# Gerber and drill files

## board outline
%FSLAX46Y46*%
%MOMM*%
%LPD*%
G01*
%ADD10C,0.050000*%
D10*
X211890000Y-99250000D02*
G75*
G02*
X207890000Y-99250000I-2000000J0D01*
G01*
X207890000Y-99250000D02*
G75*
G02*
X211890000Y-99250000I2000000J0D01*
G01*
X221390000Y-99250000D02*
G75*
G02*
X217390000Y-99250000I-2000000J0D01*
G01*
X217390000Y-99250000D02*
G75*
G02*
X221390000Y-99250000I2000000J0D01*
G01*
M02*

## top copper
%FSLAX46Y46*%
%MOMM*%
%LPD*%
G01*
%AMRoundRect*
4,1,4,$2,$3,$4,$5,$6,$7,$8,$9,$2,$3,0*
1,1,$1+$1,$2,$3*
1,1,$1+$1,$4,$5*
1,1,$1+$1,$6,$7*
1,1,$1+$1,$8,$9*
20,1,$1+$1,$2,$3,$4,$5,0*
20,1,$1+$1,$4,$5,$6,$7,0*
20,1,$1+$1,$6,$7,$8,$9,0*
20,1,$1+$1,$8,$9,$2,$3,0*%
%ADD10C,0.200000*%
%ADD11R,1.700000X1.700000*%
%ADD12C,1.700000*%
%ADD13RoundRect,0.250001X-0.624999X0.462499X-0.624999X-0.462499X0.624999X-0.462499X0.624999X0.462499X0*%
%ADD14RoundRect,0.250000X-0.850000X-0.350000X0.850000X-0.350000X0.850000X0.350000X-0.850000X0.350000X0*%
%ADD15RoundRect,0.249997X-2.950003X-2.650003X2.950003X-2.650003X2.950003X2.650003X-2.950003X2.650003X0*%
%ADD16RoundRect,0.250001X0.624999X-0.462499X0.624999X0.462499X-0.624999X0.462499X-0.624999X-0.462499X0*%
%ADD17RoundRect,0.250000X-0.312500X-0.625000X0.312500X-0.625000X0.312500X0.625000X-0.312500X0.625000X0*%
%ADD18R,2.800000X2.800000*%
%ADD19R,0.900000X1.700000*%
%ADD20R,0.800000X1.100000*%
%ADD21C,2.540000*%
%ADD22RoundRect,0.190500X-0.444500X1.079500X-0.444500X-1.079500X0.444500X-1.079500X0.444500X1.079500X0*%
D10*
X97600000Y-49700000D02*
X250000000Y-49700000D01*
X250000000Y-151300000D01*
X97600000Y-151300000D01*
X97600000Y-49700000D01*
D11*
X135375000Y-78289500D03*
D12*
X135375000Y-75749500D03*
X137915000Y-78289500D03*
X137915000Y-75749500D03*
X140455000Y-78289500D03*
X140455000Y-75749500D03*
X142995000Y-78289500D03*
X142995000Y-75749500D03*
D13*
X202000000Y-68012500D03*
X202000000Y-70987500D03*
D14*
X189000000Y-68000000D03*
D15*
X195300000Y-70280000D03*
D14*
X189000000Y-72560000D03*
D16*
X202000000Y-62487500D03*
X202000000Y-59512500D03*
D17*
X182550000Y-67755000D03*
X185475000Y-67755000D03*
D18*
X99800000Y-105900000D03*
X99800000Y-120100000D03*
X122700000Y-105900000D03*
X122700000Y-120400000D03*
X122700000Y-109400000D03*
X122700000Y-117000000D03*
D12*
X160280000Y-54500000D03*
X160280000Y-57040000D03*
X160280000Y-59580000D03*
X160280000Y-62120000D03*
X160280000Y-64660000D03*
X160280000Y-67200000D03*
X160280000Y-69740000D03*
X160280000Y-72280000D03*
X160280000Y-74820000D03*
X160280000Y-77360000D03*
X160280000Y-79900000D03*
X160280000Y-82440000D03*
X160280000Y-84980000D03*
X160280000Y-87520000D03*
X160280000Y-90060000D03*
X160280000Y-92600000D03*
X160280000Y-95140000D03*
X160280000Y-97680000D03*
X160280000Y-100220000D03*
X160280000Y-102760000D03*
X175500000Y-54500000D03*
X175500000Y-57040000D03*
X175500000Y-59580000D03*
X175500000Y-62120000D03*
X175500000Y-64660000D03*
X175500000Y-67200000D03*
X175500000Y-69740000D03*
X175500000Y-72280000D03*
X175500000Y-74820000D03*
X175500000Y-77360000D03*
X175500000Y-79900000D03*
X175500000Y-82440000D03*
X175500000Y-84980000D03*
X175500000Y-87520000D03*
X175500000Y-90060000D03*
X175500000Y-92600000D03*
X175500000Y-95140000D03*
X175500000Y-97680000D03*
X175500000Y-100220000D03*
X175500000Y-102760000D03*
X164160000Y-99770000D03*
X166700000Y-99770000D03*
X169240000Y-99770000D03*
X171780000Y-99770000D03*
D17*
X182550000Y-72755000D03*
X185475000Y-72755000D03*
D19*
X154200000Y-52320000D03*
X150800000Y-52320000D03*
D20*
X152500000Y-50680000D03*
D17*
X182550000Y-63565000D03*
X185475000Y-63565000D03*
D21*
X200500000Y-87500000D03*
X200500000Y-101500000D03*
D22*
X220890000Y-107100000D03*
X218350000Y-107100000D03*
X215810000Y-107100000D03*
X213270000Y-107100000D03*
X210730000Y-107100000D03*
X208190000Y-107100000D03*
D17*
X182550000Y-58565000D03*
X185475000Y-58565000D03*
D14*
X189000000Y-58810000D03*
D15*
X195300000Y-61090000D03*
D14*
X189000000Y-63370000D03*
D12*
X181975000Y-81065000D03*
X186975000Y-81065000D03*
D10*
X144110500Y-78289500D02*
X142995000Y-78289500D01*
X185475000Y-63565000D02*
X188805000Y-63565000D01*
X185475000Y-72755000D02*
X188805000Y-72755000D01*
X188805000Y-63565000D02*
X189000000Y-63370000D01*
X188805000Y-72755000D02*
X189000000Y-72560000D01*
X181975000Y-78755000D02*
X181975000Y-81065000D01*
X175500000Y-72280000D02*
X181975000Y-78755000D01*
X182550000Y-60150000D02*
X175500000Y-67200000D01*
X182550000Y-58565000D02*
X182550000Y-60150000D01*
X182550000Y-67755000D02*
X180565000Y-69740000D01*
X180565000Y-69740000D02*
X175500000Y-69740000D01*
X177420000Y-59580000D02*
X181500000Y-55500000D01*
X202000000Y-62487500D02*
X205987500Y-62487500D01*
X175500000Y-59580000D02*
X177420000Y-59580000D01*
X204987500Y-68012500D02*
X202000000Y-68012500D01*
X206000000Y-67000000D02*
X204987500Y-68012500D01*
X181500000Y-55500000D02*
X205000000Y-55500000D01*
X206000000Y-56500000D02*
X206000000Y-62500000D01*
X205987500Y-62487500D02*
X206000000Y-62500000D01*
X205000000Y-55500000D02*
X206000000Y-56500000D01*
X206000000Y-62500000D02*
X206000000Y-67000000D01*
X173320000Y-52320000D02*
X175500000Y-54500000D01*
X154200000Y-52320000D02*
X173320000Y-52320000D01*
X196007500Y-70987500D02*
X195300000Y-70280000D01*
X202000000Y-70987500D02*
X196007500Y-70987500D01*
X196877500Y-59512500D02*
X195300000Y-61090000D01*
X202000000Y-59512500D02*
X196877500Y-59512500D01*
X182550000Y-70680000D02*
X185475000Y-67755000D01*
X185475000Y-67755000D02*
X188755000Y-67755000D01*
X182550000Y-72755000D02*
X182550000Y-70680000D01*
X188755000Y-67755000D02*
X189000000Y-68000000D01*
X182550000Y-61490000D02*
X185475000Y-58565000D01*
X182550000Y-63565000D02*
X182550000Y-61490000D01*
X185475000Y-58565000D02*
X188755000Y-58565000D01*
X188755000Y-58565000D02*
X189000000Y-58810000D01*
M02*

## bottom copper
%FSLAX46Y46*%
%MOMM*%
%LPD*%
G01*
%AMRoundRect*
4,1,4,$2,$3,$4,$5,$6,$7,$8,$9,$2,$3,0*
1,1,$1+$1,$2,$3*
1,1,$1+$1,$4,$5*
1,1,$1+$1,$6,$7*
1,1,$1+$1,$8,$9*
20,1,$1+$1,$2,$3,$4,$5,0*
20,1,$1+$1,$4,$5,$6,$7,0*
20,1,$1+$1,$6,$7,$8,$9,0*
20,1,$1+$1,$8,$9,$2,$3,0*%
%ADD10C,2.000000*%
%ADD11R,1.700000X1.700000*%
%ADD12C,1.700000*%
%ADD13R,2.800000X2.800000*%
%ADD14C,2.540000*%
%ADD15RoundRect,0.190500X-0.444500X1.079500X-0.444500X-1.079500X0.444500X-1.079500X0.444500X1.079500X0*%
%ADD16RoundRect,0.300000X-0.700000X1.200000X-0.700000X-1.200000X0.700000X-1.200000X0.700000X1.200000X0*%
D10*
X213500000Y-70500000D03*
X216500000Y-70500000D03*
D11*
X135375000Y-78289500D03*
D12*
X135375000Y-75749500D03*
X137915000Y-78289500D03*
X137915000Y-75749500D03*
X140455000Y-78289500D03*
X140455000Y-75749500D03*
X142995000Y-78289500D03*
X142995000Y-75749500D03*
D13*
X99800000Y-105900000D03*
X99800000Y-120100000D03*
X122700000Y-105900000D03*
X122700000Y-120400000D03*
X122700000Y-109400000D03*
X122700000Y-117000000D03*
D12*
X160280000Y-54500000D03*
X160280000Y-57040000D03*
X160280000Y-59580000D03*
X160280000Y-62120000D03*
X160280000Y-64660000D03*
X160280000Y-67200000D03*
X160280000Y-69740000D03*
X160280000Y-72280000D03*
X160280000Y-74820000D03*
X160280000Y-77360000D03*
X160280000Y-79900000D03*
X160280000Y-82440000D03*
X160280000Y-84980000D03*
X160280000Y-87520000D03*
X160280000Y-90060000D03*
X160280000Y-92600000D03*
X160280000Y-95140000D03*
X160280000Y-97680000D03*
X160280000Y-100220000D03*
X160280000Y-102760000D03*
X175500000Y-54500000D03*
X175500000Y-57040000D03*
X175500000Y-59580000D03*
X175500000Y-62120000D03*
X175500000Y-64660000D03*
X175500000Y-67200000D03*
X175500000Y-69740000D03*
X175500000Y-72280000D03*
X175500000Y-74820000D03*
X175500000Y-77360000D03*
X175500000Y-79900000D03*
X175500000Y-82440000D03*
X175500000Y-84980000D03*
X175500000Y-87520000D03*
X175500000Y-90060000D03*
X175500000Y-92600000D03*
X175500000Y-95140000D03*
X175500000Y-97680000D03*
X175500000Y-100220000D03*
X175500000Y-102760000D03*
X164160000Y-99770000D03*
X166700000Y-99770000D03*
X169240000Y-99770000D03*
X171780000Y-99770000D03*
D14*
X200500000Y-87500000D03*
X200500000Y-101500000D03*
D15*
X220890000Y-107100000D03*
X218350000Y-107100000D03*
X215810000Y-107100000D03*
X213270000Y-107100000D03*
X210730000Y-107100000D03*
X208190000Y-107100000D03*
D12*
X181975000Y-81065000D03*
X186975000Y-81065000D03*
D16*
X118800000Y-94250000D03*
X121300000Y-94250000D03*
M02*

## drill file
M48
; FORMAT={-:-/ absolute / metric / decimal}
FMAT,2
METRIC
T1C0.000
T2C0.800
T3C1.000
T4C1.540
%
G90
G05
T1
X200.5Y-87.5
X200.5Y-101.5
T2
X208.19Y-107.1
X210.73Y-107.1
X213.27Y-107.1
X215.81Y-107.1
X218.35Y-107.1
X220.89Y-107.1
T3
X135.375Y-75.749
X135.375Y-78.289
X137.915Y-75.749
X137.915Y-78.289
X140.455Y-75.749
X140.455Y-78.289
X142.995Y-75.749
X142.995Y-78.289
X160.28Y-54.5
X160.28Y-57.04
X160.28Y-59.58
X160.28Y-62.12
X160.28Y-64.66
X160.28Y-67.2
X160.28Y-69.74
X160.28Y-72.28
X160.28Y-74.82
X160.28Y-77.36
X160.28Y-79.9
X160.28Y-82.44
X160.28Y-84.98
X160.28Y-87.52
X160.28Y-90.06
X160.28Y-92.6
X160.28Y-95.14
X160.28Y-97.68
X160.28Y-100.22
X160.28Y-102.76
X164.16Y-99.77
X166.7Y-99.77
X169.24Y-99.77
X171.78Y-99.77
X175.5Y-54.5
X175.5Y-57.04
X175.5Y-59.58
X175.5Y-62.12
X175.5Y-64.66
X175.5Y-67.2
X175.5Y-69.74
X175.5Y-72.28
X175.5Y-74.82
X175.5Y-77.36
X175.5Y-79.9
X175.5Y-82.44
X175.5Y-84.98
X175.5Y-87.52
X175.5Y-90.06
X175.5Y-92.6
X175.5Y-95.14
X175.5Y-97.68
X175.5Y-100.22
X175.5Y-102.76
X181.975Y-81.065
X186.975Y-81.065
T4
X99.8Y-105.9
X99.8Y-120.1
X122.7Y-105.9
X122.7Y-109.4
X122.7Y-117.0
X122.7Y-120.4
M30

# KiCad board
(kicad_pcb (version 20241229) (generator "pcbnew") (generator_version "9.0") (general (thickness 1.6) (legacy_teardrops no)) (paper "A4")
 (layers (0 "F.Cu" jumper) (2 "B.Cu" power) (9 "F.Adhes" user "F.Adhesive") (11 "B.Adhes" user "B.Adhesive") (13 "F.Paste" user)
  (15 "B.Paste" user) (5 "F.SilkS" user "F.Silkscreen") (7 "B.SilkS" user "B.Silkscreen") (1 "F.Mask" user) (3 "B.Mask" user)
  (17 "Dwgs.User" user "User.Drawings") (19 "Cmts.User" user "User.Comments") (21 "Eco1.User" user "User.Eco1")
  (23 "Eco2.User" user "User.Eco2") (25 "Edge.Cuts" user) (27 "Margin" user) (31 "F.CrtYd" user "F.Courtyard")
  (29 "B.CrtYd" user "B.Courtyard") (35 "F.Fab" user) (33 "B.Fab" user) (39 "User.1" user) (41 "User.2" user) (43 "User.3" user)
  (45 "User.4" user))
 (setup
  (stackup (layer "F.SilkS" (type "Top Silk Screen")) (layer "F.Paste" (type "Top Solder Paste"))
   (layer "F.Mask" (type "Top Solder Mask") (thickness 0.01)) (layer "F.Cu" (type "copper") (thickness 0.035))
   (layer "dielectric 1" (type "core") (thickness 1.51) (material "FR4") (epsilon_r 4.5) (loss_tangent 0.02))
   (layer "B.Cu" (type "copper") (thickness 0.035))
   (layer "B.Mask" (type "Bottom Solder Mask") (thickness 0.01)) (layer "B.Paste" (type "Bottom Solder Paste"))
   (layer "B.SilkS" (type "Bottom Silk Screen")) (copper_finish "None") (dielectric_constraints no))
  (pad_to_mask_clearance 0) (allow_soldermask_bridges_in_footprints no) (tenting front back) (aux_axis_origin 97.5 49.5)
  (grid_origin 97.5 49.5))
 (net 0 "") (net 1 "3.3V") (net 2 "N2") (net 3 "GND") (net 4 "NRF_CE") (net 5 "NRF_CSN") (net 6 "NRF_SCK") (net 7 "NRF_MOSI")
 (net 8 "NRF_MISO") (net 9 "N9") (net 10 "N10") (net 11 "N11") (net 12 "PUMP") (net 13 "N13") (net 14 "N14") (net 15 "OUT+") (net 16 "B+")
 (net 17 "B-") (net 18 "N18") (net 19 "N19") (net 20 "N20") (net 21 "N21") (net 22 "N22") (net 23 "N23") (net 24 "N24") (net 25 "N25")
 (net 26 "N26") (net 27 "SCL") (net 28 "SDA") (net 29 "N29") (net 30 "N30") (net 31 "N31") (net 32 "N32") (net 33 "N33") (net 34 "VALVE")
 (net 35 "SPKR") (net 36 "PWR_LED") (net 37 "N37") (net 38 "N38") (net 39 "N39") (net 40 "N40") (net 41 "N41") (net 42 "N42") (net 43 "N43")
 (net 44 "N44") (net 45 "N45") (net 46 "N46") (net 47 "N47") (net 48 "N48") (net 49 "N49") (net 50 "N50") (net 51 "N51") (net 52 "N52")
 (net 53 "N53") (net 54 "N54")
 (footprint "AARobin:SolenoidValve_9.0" (layer "F.Cu") (at 215 55.5)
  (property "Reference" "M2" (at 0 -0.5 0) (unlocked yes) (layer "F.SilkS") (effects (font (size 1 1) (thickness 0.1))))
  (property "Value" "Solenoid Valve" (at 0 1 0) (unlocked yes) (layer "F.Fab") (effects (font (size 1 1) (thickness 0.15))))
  (pad "1" smd circle (at -1.5 15) (size 2 2) (layers "*.Mask" "B.Cu") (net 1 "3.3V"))
  (pad "2" smd circle (at 1.5 15) (size 2 2) (layers "*.Mask" "B.Cu") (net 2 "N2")))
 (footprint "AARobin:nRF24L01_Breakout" (layer "F.Cu") (at 135.375 78.2895 90)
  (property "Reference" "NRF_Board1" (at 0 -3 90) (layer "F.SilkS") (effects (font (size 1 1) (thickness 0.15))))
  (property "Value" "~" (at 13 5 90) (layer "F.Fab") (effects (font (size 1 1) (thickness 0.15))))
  (pad "1" thru_hole rect (at 0 0 90) (size 1.7 1.7) (drill 1) (layers "*.Cu" "*.Mask") (remove_unused_layers no) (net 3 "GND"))
  (pad "2" thru_hole circle (at 2.54 0 90) (size 1.7 1.7) (drill 1) (layers "*.Cu" "*.Mask") (remove_unused_layers no) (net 1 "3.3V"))
  (pad "3" thru_hole circle (at 0 2.54 90) (size 1.7 1.7) (drill 1) (layers "*.Cu" "*.Mask") (remove_unused_layers no) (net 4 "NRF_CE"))
  (pad "4" thru_hole circle (at 2.54 2.54 90) (size 1.7 1.7) (drill 1) (layers "*.Cu" "*.Mask") (remove_unused_layers no) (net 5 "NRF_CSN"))
  (pad "5" thru_hole circle (at 0 5.08 90) (size 1.7 1.7) (drill 1) (layers "*.Cu" "*.Mask") (remove_unused_layers no) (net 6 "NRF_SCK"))
  (pad "6" thru_hole circle (at 2.54 5.08 90) (size 1.7 1.7) (drill 1) (layers "*.Cu" "*.Mask") (remove_unused_layers no) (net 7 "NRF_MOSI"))
  (pad "7" thru_hole circle (at 0 7.62 90) (size 1.7 1.7) (drill 1) (layers "*.Cu" "*.Mask") (remove_unused_layers no) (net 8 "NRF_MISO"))
  (pad "8" thru_hole circle (at 2.54 7.62 90) (size 1.7 1.7) (drill 1) (layers "*.Cu" "*.Mask") (remove_unused_layers no) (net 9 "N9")))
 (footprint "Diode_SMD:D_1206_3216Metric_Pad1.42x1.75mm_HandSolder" (layer "F.Cu") (at 202 69.5 -90)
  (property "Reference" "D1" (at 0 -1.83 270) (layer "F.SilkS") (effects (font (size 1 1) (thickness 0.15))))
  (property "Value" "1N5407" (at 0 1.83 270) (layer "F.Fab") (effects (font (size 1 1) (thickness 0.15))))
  (pad "1" smd roundrect (at -1.4875 0 270) (size 1.425 1.75) (layers "F.Cu" "F.Mask" "F.Paste") (roundrect_rratio 0.175439) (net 1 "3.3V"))
  (pad "2" smd roundrect (at 1.4875 0 270) (size 1.425 1.75) (layers "F.Cu" "F.Mask" "F.Paste") (roundrect_rratio 0.175439) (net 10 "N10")))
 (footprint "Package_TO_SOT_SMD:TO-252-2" (layer "F.Cu") (at 194.04 70.28)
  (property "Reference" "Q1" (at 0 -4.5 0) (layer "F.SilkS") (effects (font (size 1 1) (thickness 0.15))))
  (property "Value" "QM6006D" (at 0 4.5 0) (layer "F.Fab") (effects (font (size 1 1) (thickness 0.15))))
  (pad "" smd roundrect (at -0.415 -1.525) (size 3.05 2.75) (layers "F.Paste") (roundrect_rratio 0.090909))
  (pad "" smd roundrect (at -0.415 1.525) (size 3.05 2.75) (layers "F.Paste") (roundrect_rratio 0.090909))
  (pad "" smd roundrect (at 2.935 -1.525) (size 3.05 2.75) (layers "F.Paste") (roundrect_rratio 0.090909))
  (pad "" smd roundrect (at 2.935 1.525) (size 3.05 2.75) (layers "F.Paste") (roundrect_rratio 0.090909))
  (pad "1" smd roundrect (at -5.04 -2.28) (size 2.2 1.2) (layers "F.Cu" "F.Mask" "F.Paste") (roundrect_rratio 0.208333) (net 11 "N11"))
  (pad "2" smd roundrect (at 1.26 0) (size 6.4 5.8) (layers "F.Cu" "F.Mask") (roundrect_rratio 0.043103) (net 10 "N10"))
  (pad "3" smd roundrect (at -5.04 2.28) (size 2.2 1.2) (layers "F.Cu" "F.Mask" "F.Paste") (roundrect_rratio 0.208333) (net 3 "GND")))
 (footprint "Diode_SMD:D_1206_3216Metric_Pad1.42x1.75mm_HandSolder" (layer "F.Cu") (at 202 61 90)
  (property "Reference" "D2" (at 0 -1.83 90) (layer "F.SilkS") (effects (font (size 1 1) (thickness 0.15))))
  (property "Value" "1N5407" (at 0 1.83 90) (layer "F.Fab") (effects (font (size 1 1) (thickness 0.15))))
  (pad "1" smd roundrect (at -1.4875 0 90) (size 1.425 1.75) (layers "F.Cu" "F.Mask" "F.Paste") (roundrect_rratio 0.175439) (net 1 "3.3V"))
  (pad "2" smd roundrect (at 1.4875 0 90) (size 1.425 1.75) (layers "F.Cu" "F.Mask" "F.Paste") (roundrect_rratio 0.175439) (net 2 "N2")))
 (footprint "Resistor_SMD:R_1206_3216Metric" (layer "F.Cu") (at 184.0125 67.755)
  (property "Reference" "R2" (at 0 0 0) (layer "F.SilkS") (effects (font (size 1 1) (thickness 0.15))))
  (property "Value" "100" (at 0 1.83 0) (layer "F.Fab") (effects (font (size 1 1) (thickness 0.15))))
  (pad "1" smd roundrect (at -1.4625 0) (size 1.125 1.75) (layers "F.Cu" "F.Mask" "F.Paste") (roundrect_rratio 0.222222) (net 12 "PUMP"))
  (pad "2" smd roundrect (at 1.4625 0) (size 1.125 1.75) (layers "F.Cu" "F.Mask" "F.Paste") (roundrect_rratio 0.222222) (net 11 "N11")))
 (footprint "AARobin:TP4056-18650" (layer "F.Cu") (at 111.8 113.5)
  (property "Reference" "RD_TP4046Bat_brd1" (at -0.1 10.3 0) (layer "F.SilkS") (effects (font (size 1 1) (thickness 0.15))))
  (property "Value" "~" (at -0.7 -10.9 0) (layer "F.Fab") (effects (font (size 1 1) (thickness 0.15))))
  (pad "1" thru_hole rect (at -12 -7.6) (size 2.8 2.8) (drill 1.54) (layers "*.Cu" "*.Mask") (remove_unused_layers no) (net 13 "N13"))
  (pad "2" thru_hole rect (at -12 6.6) (size 2.8 2.8) (drill 1.54) (layers "*.Cu" "*.Mask") (remove_unused_layers no) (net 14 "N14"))
  (pad "3" thru_hole rect (at 10.9 -7.6) (size 2.8 2.8) (drill 1.54) (layers "*.Cu" "*.Mask") (remove_unused_layers no) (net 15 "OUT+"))
  (pad "4" thru_hole rect (at 10.9 6.9) (size 2.8 2.8) (drill 1.54) (layers "*.Cu" "*.Mask") (remove_unused_layers no) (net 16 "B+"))
  (pad "5" thru_hole rect (at 10.9 -4.1) (size 2.8 2.8) (drill 1.54) (layers "*.Cu" "*.Mask") (remove_unused_layers no) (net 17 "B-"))
  (pad "6" thru_hole rect (at 10.9 3.5) (size 2.8 2.8) (drill 1.54) (layers "*.Cu" "*.Mask") (remove_unused_layers no) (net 3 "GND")))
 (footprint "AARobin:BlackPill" (layer "F.Cu") (at 168.13 78.365)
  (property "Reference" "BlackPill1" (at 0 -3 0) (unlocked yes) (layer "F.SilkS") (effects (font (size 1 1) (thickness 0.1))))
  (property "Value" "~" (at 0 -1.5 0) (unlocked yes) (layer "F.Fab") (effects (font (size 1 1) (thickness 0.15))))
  (pad "1" thru_hole circle (at -7.85 -23.865) (size 1.7 1.7) (drill 1) (layers "*.Cu" "*.Mask") (remove_unused_layers no) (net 4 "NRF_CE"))
  (pad "2" thru_hole circle (at -7.85 -21.325) (size 1.7 1.7) (drill 1) (layers "*.Cu" "*.Mask") (remove_unused_layers no) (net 6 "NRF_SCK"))
  (pad "3" thru_hole circle (at -7.85 -18.785) (size 1.7 1.7) (drill 1) (layers "*.Cu" "*.Mask") (remove_unused_layers no)
   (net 7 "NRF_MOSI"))
  (pad "4" thru_hole circle (at -7.85 -16.245) (size 1.7 1.7) (drill 1) (layers "*.Cu" "*.Mask") (remove_unused_layers no)
   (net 8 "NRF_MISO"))
  (pad "5" thru_hole circle (at -7.85 -13.705) (size 1.7 1.7) (drill 1) (layers "*.Cu" "*.Mask") (remove_unused_layers no) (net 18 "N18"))
  (pad "6" thru_hole circle (at -7.85 -11.165) (size 1.7 1.7) (drill 1) (layers "*.Cu" "*.Mask") (remove_unused_layers no) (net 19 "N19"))
  (pad "7" thru_hole circle (at -7.85 -8.625) (size 1.7 1.7) (drill 1) (layers "*.Cu" "*.Mask") (remove_unused_layers no) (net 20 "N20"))
  (pad "8" thru_hole circle (at -7.85 -6.085) (size 1.7 1.7) (drill 1) (layers "*.Cu" "*.Mask") (remove_unused_layers no) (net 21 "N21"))
  (pad "9" thru_hole circle (at -7.85 -3.545) (size 1.7 1.7) (drill 1) (layers "*.Cu" "*.Mask") (remove_unused_layers no) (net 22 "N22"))
  (pad "10" thru_hole circle (at -7.85 -1.005) (size 1.7 1.7) (drill 1) (layers "*.Cu" "*.Mask") (remove_unused_layers no) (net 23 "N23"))
  (pad "11" thru_hole circle (at -7.85 1.535) (size 1.7 1.7) (drill 1) (layers "*.Cu" "*.Mask") (remove_unused_layers no) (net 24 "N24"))
  (pad "12" thru_hole circle (at -7.85 4.075) (size 1.7 1.7) (drill 1) (layers "*.Cu" "*.Mask") (remove_unused_layers no) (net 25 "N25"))
  (pad "13" thru_hole circle (at -7.85 6.615) (size 1.7 1.7) (drill 1) (layers "*.Cu" "*.Mask") (remove_unused_layers no) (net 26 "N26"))
  (pad "14" thru_hole circle (at -7.85 9.155) (size 1.7 1.7) (drill 1) (layers "*.Cu" "*.Mask") (remove_unused_layers no) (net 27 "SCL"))
  (pad "15" thru_hole circle (at -7.85 11.695) (size 1.7 1.7) (drill 1) (layers "*.Cu" "*.Mask") (remove_unused_layers no) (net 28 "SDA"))
  (pad "16" thru_hole circle (at -7.85 14.235) (size 1.7 1.7) (drill 1) (layers "*.Cu" "*.Mask") (remove_unused_layers no) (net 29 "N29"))
  (pad "17" thru_hole circle (at -7.85 16.775) (size 1.7 1.7) (drill 1) (layers "*.Cu" "*.Mask") (remove_unused_layers no) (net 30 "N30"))
  (pad "18" thru_hole circle (at -7.85 19.315) (size 1.7 1.7) (drill 1) (layers "*.Cu" "*.Mask") (remove_unused_layers no) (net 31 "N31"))
  (pad "19" thru_hole circle (at -7.85 21.855) (size 1.7 1.7) (drill 1) (layers "*.Cu" "*.Mask") (remove_unused_layers no) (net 3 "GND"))
  (pad "20" thru_hole circle (at -7.85 24.395) (size 1.7 1.7) (drill 1) (layers "*.Cu" "*.Mask") (remove_unused_layers no) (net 1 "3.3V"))
  (pad "21" thru_hole circle (at 7.37 -23.865) (size 1.7 1.7) (drill 1) (layers "*.Cu" "*.Mask") (remove_unused_layers no) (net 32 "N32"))
  (pad "22" thru_hole circle (at 7.37 -21.325) (size 1.7 1.7) (drill 1) (layers "*.Cu" "*.Mask") (remove_unused_layers no) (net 3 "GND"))
  (pad "23" thru_hole circle (at 7.37 -18.785) (size 1.7 1.7) (drill 1) (layers "*.Cu" "*.Mask") (remove_unused_layers no) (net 1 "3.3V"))
  (pad "24" thru_hole circle (at 7.37 -16.245) (size 1.7 1.7) (drill 1) (layers "*.Cu" "*.Mask") (remove_unused_layers no) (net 6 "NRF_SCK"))
  (pad "25" thru_hole circle (at 7.37 -13.705) (size 1.7 1.7) (drill 1) (layers "*.Cu" "*.Mask") (remove_unused_layers no) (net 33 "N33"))
  (pad "26" thru_hole circle (at 7.37 -11.165) (size 1.7 1.7) (drill 1) (layers "*.Cu" "*.Mask") (remove_unused_layers no) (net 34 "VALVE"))
  (pad "27" thru_hole circle (at 7.37 -8.625) (size 1.7 1.7) (drill 1) (layers "*.Cu" "*.Mask") (remove_unused_layers no) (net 12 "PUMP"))
  (pad "28" thru_hole circle (at 7.37 -6.085) (size 1.7 1.7) (drill 1) (layers "*.Cu" "*.Mask") (remove_unused_layers no) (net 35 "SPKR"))
  (pad "29" thru_hole circle (at 7.37 -3.545) (size 1.7 1.7) (drill 1) (layers "*.Cu" "*.Mask") (remove_unused_layers no) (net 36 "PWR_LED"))
  (pad "30" thru_hole circle (at 7.37 -1.005) (size 1.7 1.7) (drill 1) (layers "*.Cu" "*.Mask") (remove_unused_layers no) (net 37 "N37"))
  (pad "31" thru_hole circle (at 7.37 1.535) (size 1.7 1.7) (drill 1) (layers "*.Cu" "*.Mask") (remove_unused_layers no) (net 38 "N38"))
  (pad "32" thru_hole circle (at 7.37 4.075) (size 1.7 1.7) (drill 1) (layers "*.Cu" "*.Mask") (remove_unused_layers no) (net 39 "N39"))
  (pad "33" thru_hole circle (at 7.37 6.615) (size 1.7 1.7) (drill 1) (layers "*.Cu" "*.Mask") (remove_unused_layers no) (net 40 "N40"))
  (pad "34" thru_hole circle (at 7.37 9.155) (size 1.7 1.7) (drill 1) (layers "*.Cu" "*.Mask") (remove_unused_layers no) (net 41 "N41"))
  (pad "35" thru_hole circle (at 7.37 11.695) (size 1.7 1.7) (drill 1) (layers "*.Cu" "*.Mask") (remove_unused_layers no) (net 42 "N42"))
  (pad "36" thru_hole circle (at 7.37 14.235) (size 1.7 1.7) (drill 1) (layers "*.Cu" "*.Mask") (remove_unused_layers no) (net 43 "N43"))
  (pad "37" thru_hole circle (at 7.37 16.775) (size 1.7 1.7) (drill 1) (layers "*.Cu" "*.Mask") (remove_unused_layers no) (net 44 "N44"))
  (pad "38" thru_hole circle (at 7.37 19.315) (size 1.7 1.7) (drill 1) (layers "*.Cu" "*.Mask") (remove_unused_layers no) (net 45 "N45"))
  (pad "39" thru_hole circle (at 7.37 21.855) (size 1.7 1.7) (drill 1) (layers "*.Cu" "*.Mask") (remove_unused_layers no) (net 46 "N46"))
  (pad "40" thru_hole circle (at 7.37 24.395) (size 1.7 1.7) (drill 1) (layers "*.Cu" "*.Mask") (remove_unused_layers no) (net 16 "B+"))
  (pad "41" thru_hole circle (at -3.97 21.405) (size 1.7 1.7) (drill 1) (layers "*.Cu" "*.Mask") (remove_unused_layers no) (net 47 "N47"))
  (pad "42" thru_hole circle (at -1.43 21.405) (size 1.7 1.7) (drill 1) (layers "*.Cu" "*.Mask") (remove_unused_layers no) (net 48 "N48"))
  (pad "43" thru_hole circle (at 1.11 21.405) (size 1.7 1.7) (drill 1) (layers "*.Cu" "*.Mask") (remove_unused_layers no) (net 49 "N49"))
  (pad "44" thru_hole circle (at 3.65 21.405) (size 1.7 1.7) (drill 1) (layers "*.Cu" "*.Mask") (remove_unused_layers no) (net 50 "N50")))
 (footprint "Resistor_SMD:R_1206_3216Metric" (layer "F.Cu") (at 184.0125 72.755)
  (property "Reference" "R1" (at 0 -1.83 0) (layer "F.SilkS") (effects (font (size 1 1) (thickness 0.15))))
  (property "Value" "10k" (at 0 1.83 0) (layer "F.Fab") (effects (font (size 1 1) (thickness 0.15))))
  (pad "1" smd roundrect (at -1.4625 0) (size 1.125 1.75) (layers "F.Cu" "F.Mask" "F.Paste") (roundrect_rratio 0.222222) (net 11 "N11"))
  (pad "2" smd roundrect (at 1.4625 0) (size 1.125 1.75) (layers "F.Cu" "F.Mask" "F.Paste") (roundrect_rratio 0.222222) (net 3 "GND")))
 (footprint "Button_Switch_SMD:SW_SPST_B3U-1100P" (layer "F.Cu") (at 152.5 51.5 180)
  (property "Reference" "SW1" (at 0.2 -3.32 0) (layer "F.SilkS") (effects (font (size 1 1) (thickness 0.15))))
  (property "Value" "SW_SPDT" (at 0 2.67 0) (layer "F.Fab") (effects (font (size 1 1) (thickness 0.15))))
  (pad "1" smd rect (at -1.7 -0.82 180) (size 0.9 1.7) (layers "F.Cu" "F.Mask" "F.Paste") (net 32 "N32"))
  (pad "2" smd rect (at 1.7 -0.82 180) (size 0.9 1.7) (layers "F.Cu" "F.Mask" "F.Paste") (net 15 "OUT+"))
  (pad "3" smd rect (at 0 0.82 180) (size 0.8 1.1) (layers "F.Cu" "F.Mask" "F.Paste") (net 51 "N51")))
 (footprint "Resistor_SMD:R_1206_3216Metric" (layer "F.Cu") (at 184.0125 63.565)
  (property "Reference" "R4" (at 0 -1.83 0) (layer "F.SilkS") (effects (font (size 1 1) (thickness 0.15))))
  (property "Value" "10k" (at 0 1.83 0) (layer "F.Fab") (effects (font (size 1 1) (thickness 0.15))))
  (pad "1" smd roundrect (at -1.4625 0) (size 1.125 1.75) (layers "F.Cu" "F.Mask" "F.Paste") (roundrect_rratio 0.222222) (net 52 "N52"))
  (pad "2" smd roundrect (at 1.4625 0) (size 1.125 1.75) (layers "F.Cu" "F.Mask" "F.Paste") (roundrect_rratio 0.222222) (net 3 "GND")))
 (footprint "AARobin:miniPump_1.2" (layer "F.Cu") (at 244.5 94.5 -90)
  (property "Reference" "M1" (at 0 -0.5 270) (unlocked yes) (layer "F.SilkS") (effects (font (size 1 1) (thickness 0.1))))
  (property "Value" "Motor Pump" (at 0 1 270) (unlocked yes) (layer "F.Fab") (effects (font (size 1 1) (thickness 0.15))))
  (pad "1" thru_hole circle (at -7 44 270) (size 2.54 2.54) (drill 0.000001) (layers "*.Cu" "*.Mask") (remove_unused_layers no)
   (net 1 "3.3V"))
  (pad "2" thru_hole circle (at 7 44 270) (size 2.54 2.54) (drill 0.000001) (layers "*.Cu" "*.Mask") (remove_unused_layers no)
   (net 10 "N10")))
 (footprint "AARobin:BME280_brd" (layer "F.Cu") (at 214.64 102.5 -90)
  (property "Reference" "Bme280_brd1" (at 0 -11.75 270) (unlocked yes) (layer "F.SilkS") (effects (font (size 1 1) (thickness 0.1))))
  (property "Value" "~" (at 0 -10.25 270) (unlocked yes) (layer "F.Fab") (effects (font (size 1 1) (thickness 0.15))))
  (fp_circle (center -3.25 4.75) (end -1.25 4.75) (stroke (width 0.05) (type default)) (fill no) (layer "Edge.Cuts"))
  (fp_circle (center -3.25 -4.75) (end -1.25 -4.75) (stroke (width 0.05) (type default)) (fill no) (layer "Edge.Cuts"))
  (pad "1" thru_hole roundrect (at 4.6 -6.25 270) (size 2.54 1.27) (drill 0.8) (layers "*.Cu" "*.Mask") (remove_unused_layers no)
   (roundrect_rratio 0.15) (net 1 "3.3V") (thermal_bridge_angle 45))
  (pad "2" thru_hole roundrect (at 4.6 -3.71 270) (size 2.54 1.27) (drill 0.8) (layers "*.Cu" "*.Mask") (remove_unused_layers no)
   (roundrect_rratio 0.15) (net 3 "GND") (thermal_bridge_angle 45))
  (pad "3" thru_hole roundrect (at 4.6 -1.17 270) (size 2.54 1.27) (drill 0.8) (layers "*.Cu" "*.Mask") (remove_unused_layers no)
   (roundrect_rratio 0.15) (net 27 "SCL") (thermal_bridge_angle 45))
  (pad "4" thru_hole roundrect (at 4.6 1.37 270) (size 2.54 1.27) (drill 0.8) (layers "*.Cu" "*.Mask") (remove_unused_layers no)
   (roundrect_rratio 0.15) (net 28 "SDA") (thermal_bridge_angle 45))
  (pad "5" thru_hole roundrect (at 4.6 3.91 270) (size 2.54 1.27) (drill 0.8) (layers "*.Cu" "*.Mask") (remove_unused_layers no)
   (roundrect_rratio 0.15) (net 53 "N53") (thermal_bridge_angle 45))
  (pad "6" thru_hole roundrect (at 4.6 6.45 270) (size 2.54 1.27) (drill 0.8) (layers "*.Cu" "*.Mask") (remove_unused_layers no)
   (roundrect_rratio 0.15) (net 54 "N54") (thermal_bridge_angle 45)))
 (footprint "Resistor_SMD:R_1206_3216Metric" (layer "F.Cu") (at 184.0125 58.565)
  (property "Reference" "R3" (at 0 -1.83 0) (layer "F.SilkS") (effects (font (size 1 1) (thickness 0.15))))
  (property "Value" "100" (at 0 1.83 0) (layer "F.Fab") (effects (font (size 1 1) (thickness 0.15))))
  (pad "1" smd roundrect (at -1.4625 0) (size 1.125 1.75) (layers "F.Cu" "F.Mask" "F.Paste") (roundrect_rratio 0.222222) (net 34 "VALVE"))
  (pad "2" smd roundrect (at 1.4625 0) (size 1.125 1.75) (layers "F.Cu" "F.Mask" "F.Paste") (roundrect_rratio 0.222222) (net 52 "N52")))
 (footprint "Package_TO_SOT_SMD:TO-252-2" (layer "F.Cu") (at 194.04 61.09)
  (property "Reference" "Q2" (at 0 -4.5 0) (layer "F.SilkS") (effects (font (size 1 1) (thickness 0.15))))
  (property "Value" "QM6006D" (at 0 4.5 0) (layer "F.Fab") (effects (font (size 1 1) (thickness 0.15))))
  (pad "" smd roundrect (at -0.415 -1.525) (size 3.05 2.75) (layers "F.Paste") (roundrect_rratio 0.090909))
  (pad "" smd roundrect (at -0.415 1.525) (size 3.05 2.75) (layers "F.Paste") (roundrect_rratio 0.090909))
  (pad "" smd roundrect (at 2.935 -1.525) (size 3.05 2.75) (layers "F.Paste") (roundrect_rratio 0.090909))
  (pad "" smd roundrect (at 2.935 1.525) (size 3.05 2.75) (layers "F.Paste") (roundrect_rratio 0.090909))
  (pad "1" smd roundrect (at -5.04 -2.28) (size 2.2 1.2) (layers "F.Cu" "F.Mask" "F.Paste") (roundrect_rratio 0.208333) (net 52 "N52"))
  (pad "2" smd roundrect (at 1.26 0) (size 6.4 5.8) (layers "F.Cu" "F.Mask") (roundrect_rratio 0.043103) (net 2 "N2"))
  (pad "3" smd roundrect (at -5.04 2.28) (size 2.2 1.2) (layers "F.Cu" "F.Mask" "F.Paste") (roundrect_rratio 0.208333) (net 3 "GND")))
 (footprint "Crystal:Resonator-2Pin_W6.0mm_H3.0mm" (layer "F.Cu") (at 181.975 81.065)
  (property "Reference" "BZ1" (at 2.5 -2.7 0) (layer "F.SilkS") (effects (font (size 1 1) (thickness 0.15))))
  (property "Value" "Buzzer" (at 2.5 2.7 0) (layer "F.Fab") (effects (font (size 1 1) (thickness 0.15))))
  (pad "1" thru_hole circle (at 0 0) (size 1.7 1.7) (drill 1) (layers "*.Cu" "*.Mask") (remove_unused_layers no) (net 35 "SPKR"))
  (pad "2" thru_hole circle (at 5 0) (size 1.7 1.7) (drill 1) (layers "*.Cu" "*.Mask") (remove_unused_layers no) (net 3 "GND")))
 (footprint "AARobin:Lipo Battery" (layer "B.Cu") (at 113.05 76 -90)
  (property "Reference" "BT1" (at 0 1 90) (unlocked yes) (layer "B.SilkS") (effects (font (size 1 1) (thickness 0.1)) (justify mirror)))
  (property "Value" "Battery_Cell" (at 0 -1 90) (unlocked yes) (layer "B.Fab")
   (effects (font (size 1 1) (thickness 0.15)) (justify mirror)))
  (pad "1" smd roundrect (at 18.25 -5.75 270) (size 3 2) (layers "B.Cu") (roundrect_rratio 0.15) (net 16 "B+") (thermal_bridge_angle 45))
  (pad "2" smd roundrect (at 18.25 -8.25 270) (size 3 2) (layers "B.Cu" "B.Mask" "B.Paste") (roundrect_rratio 0.15) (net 17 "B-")
   (thermal_bridge_angle 45)))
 (gr_rect (start 97.6 49.7) (end 250 151.3) (stroke (width 0.2) (type solid)) (fill no) (layer "F.Cu") (net 1))
 (segment (start 144.1105 78.2895) (end 142.995 78.2895) (width 0.2) (layer "F.Cu") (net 8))
 (segment (start 185.475 63.565) (end 188.805 63.565) (width 0.2) (layer "F.Cu") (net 3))
 (segment (start 185.475 72.755) (end 188.805 72.755) (width 0.2) (layer "F.Cu") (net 3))
 (segment (start 188.805 63.565) (end 189 63.37) (width 0.2) (layer "F.Cu") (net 3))
 (segment (start 188.805 72.755) (end 189 72.56) (width 0.2) (layer "F.Cu") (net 3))
 (segment (start 181.975 78.755) (end 181.975 81.065) (width 0.2) (layer "F.Cu") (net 35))
 (segment (start 175.5 72.28) (end 181.975 78.755) (width 0.2) (layer "F.Cu") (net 35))
 (segment (start 182.55 60.15) (end 175.5 67.2) (width 0.2) (layer "F.Cu") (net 34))
 (segment (start 182.55 58.565) (end 182.55 60.15) (width 0.2) (layer "F.Cu") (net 34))
 (segment (start 182.55 67.755) (end 180.565 69.74) (width 0.2) (layer "F.Cu") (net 12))
 (segment (start 180.565 69.74) (end 175.5 69.74) (width 0.2) (layer "F.Cu") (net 12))
 (segment (start 177.42 59.58) (end 181.5 55.5) (width 0.2) (layer "F.Cu") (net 1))
 (segment (start 202 62.4875) (end 205.9875 62.4875) (width 0.2) (layer "F.Cu") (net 1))
 (segment (start 175.5 59.58) (end 177.42 59.58) (width 0.2) (layer "F.Cu") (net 1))
 (segment (start 204.9875 68.0125) (end 202 68.0125) (width 0.2) (layer "F.Cu") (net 1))
 (segment (start 206 67) (end 204.9875 68.0125) (width 0.2) (layer "F.Cu") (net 1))
 (segment (start 181.5 55.5) (end 205 55.5) (width 0.2) (layer "F.Cu") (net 1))
 (segment (start 206 56.5) (end 206 62.5) (width 0.2) (layer "F.Cu") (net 1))
 (segment (start 205.9875 62.4875) (end 206 62.5) (width 0.2) (layer "F.Cu") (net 1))
 (segment (start 205 55.5) (end 206 56.5) (width 0.2) (layer "F.Cu") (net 1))
 (segment (start 206 62.5) (end 206 67) (width 0.2) (layer "F.Cu") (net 1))
 (segment (start 173.32 52.32) (end 175.5 54.5) (width 0.2) (layer "F.Cu") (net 32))
 (segment (start 154.2 52.32) (end 173.32 52.32) (width 0.2) (layer "F.Cu") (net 32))
 (segment (start 196.0075 70.9875) (end 195.3 70.28) (width 0.2) (layer "F.Cu") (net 10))
 (segment (start 202 70.9875) (end 196.0075 70.9875) (width 0.2) (layer "F.Cu") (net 10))
 (segment (start 196.8775 59.5125) (end 195.3 61.09) (width 0.2) (layer "F.Cu") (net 2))
 (segment (start 202 59.5125) (end 196.8775 59.5125) (width 0.2) (layer "F.Cu") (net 2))
 (segment (start 182.55 70.68) (end 185.475 67.755) (width 0.2) (layer "F.Cu") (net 11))
 (segment (start 185.475 67.755) (end 188.755 67.755) (width 0.2) (layer "F.Cu") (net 11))
 (segment (start 182.55 72.755) (end 182.55 70.68) (width 0.2) (layer "F.Cu") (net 11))
 (segment (start 188.755 67.755) (end 189 68) (width 0.2) (layer "F.Cu") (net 11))
 (segment (start 182.55 61.49) (end 185.475 58.565) (width 0.2) (layer "F.Cu") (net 52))
 (segment (start 182.55 63.565) (end 182.55 61.49) (width 0.2) (layer "F.Cu") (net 52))
 (segment (start 185.475 58.565) (end 188.755 58.565) (width 0.2) (layer "F.Cu") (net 52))
 (segment (start 188.755 58.565) (end 189 58.81) (width 0.2) (layer "F.Cu") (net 52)))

